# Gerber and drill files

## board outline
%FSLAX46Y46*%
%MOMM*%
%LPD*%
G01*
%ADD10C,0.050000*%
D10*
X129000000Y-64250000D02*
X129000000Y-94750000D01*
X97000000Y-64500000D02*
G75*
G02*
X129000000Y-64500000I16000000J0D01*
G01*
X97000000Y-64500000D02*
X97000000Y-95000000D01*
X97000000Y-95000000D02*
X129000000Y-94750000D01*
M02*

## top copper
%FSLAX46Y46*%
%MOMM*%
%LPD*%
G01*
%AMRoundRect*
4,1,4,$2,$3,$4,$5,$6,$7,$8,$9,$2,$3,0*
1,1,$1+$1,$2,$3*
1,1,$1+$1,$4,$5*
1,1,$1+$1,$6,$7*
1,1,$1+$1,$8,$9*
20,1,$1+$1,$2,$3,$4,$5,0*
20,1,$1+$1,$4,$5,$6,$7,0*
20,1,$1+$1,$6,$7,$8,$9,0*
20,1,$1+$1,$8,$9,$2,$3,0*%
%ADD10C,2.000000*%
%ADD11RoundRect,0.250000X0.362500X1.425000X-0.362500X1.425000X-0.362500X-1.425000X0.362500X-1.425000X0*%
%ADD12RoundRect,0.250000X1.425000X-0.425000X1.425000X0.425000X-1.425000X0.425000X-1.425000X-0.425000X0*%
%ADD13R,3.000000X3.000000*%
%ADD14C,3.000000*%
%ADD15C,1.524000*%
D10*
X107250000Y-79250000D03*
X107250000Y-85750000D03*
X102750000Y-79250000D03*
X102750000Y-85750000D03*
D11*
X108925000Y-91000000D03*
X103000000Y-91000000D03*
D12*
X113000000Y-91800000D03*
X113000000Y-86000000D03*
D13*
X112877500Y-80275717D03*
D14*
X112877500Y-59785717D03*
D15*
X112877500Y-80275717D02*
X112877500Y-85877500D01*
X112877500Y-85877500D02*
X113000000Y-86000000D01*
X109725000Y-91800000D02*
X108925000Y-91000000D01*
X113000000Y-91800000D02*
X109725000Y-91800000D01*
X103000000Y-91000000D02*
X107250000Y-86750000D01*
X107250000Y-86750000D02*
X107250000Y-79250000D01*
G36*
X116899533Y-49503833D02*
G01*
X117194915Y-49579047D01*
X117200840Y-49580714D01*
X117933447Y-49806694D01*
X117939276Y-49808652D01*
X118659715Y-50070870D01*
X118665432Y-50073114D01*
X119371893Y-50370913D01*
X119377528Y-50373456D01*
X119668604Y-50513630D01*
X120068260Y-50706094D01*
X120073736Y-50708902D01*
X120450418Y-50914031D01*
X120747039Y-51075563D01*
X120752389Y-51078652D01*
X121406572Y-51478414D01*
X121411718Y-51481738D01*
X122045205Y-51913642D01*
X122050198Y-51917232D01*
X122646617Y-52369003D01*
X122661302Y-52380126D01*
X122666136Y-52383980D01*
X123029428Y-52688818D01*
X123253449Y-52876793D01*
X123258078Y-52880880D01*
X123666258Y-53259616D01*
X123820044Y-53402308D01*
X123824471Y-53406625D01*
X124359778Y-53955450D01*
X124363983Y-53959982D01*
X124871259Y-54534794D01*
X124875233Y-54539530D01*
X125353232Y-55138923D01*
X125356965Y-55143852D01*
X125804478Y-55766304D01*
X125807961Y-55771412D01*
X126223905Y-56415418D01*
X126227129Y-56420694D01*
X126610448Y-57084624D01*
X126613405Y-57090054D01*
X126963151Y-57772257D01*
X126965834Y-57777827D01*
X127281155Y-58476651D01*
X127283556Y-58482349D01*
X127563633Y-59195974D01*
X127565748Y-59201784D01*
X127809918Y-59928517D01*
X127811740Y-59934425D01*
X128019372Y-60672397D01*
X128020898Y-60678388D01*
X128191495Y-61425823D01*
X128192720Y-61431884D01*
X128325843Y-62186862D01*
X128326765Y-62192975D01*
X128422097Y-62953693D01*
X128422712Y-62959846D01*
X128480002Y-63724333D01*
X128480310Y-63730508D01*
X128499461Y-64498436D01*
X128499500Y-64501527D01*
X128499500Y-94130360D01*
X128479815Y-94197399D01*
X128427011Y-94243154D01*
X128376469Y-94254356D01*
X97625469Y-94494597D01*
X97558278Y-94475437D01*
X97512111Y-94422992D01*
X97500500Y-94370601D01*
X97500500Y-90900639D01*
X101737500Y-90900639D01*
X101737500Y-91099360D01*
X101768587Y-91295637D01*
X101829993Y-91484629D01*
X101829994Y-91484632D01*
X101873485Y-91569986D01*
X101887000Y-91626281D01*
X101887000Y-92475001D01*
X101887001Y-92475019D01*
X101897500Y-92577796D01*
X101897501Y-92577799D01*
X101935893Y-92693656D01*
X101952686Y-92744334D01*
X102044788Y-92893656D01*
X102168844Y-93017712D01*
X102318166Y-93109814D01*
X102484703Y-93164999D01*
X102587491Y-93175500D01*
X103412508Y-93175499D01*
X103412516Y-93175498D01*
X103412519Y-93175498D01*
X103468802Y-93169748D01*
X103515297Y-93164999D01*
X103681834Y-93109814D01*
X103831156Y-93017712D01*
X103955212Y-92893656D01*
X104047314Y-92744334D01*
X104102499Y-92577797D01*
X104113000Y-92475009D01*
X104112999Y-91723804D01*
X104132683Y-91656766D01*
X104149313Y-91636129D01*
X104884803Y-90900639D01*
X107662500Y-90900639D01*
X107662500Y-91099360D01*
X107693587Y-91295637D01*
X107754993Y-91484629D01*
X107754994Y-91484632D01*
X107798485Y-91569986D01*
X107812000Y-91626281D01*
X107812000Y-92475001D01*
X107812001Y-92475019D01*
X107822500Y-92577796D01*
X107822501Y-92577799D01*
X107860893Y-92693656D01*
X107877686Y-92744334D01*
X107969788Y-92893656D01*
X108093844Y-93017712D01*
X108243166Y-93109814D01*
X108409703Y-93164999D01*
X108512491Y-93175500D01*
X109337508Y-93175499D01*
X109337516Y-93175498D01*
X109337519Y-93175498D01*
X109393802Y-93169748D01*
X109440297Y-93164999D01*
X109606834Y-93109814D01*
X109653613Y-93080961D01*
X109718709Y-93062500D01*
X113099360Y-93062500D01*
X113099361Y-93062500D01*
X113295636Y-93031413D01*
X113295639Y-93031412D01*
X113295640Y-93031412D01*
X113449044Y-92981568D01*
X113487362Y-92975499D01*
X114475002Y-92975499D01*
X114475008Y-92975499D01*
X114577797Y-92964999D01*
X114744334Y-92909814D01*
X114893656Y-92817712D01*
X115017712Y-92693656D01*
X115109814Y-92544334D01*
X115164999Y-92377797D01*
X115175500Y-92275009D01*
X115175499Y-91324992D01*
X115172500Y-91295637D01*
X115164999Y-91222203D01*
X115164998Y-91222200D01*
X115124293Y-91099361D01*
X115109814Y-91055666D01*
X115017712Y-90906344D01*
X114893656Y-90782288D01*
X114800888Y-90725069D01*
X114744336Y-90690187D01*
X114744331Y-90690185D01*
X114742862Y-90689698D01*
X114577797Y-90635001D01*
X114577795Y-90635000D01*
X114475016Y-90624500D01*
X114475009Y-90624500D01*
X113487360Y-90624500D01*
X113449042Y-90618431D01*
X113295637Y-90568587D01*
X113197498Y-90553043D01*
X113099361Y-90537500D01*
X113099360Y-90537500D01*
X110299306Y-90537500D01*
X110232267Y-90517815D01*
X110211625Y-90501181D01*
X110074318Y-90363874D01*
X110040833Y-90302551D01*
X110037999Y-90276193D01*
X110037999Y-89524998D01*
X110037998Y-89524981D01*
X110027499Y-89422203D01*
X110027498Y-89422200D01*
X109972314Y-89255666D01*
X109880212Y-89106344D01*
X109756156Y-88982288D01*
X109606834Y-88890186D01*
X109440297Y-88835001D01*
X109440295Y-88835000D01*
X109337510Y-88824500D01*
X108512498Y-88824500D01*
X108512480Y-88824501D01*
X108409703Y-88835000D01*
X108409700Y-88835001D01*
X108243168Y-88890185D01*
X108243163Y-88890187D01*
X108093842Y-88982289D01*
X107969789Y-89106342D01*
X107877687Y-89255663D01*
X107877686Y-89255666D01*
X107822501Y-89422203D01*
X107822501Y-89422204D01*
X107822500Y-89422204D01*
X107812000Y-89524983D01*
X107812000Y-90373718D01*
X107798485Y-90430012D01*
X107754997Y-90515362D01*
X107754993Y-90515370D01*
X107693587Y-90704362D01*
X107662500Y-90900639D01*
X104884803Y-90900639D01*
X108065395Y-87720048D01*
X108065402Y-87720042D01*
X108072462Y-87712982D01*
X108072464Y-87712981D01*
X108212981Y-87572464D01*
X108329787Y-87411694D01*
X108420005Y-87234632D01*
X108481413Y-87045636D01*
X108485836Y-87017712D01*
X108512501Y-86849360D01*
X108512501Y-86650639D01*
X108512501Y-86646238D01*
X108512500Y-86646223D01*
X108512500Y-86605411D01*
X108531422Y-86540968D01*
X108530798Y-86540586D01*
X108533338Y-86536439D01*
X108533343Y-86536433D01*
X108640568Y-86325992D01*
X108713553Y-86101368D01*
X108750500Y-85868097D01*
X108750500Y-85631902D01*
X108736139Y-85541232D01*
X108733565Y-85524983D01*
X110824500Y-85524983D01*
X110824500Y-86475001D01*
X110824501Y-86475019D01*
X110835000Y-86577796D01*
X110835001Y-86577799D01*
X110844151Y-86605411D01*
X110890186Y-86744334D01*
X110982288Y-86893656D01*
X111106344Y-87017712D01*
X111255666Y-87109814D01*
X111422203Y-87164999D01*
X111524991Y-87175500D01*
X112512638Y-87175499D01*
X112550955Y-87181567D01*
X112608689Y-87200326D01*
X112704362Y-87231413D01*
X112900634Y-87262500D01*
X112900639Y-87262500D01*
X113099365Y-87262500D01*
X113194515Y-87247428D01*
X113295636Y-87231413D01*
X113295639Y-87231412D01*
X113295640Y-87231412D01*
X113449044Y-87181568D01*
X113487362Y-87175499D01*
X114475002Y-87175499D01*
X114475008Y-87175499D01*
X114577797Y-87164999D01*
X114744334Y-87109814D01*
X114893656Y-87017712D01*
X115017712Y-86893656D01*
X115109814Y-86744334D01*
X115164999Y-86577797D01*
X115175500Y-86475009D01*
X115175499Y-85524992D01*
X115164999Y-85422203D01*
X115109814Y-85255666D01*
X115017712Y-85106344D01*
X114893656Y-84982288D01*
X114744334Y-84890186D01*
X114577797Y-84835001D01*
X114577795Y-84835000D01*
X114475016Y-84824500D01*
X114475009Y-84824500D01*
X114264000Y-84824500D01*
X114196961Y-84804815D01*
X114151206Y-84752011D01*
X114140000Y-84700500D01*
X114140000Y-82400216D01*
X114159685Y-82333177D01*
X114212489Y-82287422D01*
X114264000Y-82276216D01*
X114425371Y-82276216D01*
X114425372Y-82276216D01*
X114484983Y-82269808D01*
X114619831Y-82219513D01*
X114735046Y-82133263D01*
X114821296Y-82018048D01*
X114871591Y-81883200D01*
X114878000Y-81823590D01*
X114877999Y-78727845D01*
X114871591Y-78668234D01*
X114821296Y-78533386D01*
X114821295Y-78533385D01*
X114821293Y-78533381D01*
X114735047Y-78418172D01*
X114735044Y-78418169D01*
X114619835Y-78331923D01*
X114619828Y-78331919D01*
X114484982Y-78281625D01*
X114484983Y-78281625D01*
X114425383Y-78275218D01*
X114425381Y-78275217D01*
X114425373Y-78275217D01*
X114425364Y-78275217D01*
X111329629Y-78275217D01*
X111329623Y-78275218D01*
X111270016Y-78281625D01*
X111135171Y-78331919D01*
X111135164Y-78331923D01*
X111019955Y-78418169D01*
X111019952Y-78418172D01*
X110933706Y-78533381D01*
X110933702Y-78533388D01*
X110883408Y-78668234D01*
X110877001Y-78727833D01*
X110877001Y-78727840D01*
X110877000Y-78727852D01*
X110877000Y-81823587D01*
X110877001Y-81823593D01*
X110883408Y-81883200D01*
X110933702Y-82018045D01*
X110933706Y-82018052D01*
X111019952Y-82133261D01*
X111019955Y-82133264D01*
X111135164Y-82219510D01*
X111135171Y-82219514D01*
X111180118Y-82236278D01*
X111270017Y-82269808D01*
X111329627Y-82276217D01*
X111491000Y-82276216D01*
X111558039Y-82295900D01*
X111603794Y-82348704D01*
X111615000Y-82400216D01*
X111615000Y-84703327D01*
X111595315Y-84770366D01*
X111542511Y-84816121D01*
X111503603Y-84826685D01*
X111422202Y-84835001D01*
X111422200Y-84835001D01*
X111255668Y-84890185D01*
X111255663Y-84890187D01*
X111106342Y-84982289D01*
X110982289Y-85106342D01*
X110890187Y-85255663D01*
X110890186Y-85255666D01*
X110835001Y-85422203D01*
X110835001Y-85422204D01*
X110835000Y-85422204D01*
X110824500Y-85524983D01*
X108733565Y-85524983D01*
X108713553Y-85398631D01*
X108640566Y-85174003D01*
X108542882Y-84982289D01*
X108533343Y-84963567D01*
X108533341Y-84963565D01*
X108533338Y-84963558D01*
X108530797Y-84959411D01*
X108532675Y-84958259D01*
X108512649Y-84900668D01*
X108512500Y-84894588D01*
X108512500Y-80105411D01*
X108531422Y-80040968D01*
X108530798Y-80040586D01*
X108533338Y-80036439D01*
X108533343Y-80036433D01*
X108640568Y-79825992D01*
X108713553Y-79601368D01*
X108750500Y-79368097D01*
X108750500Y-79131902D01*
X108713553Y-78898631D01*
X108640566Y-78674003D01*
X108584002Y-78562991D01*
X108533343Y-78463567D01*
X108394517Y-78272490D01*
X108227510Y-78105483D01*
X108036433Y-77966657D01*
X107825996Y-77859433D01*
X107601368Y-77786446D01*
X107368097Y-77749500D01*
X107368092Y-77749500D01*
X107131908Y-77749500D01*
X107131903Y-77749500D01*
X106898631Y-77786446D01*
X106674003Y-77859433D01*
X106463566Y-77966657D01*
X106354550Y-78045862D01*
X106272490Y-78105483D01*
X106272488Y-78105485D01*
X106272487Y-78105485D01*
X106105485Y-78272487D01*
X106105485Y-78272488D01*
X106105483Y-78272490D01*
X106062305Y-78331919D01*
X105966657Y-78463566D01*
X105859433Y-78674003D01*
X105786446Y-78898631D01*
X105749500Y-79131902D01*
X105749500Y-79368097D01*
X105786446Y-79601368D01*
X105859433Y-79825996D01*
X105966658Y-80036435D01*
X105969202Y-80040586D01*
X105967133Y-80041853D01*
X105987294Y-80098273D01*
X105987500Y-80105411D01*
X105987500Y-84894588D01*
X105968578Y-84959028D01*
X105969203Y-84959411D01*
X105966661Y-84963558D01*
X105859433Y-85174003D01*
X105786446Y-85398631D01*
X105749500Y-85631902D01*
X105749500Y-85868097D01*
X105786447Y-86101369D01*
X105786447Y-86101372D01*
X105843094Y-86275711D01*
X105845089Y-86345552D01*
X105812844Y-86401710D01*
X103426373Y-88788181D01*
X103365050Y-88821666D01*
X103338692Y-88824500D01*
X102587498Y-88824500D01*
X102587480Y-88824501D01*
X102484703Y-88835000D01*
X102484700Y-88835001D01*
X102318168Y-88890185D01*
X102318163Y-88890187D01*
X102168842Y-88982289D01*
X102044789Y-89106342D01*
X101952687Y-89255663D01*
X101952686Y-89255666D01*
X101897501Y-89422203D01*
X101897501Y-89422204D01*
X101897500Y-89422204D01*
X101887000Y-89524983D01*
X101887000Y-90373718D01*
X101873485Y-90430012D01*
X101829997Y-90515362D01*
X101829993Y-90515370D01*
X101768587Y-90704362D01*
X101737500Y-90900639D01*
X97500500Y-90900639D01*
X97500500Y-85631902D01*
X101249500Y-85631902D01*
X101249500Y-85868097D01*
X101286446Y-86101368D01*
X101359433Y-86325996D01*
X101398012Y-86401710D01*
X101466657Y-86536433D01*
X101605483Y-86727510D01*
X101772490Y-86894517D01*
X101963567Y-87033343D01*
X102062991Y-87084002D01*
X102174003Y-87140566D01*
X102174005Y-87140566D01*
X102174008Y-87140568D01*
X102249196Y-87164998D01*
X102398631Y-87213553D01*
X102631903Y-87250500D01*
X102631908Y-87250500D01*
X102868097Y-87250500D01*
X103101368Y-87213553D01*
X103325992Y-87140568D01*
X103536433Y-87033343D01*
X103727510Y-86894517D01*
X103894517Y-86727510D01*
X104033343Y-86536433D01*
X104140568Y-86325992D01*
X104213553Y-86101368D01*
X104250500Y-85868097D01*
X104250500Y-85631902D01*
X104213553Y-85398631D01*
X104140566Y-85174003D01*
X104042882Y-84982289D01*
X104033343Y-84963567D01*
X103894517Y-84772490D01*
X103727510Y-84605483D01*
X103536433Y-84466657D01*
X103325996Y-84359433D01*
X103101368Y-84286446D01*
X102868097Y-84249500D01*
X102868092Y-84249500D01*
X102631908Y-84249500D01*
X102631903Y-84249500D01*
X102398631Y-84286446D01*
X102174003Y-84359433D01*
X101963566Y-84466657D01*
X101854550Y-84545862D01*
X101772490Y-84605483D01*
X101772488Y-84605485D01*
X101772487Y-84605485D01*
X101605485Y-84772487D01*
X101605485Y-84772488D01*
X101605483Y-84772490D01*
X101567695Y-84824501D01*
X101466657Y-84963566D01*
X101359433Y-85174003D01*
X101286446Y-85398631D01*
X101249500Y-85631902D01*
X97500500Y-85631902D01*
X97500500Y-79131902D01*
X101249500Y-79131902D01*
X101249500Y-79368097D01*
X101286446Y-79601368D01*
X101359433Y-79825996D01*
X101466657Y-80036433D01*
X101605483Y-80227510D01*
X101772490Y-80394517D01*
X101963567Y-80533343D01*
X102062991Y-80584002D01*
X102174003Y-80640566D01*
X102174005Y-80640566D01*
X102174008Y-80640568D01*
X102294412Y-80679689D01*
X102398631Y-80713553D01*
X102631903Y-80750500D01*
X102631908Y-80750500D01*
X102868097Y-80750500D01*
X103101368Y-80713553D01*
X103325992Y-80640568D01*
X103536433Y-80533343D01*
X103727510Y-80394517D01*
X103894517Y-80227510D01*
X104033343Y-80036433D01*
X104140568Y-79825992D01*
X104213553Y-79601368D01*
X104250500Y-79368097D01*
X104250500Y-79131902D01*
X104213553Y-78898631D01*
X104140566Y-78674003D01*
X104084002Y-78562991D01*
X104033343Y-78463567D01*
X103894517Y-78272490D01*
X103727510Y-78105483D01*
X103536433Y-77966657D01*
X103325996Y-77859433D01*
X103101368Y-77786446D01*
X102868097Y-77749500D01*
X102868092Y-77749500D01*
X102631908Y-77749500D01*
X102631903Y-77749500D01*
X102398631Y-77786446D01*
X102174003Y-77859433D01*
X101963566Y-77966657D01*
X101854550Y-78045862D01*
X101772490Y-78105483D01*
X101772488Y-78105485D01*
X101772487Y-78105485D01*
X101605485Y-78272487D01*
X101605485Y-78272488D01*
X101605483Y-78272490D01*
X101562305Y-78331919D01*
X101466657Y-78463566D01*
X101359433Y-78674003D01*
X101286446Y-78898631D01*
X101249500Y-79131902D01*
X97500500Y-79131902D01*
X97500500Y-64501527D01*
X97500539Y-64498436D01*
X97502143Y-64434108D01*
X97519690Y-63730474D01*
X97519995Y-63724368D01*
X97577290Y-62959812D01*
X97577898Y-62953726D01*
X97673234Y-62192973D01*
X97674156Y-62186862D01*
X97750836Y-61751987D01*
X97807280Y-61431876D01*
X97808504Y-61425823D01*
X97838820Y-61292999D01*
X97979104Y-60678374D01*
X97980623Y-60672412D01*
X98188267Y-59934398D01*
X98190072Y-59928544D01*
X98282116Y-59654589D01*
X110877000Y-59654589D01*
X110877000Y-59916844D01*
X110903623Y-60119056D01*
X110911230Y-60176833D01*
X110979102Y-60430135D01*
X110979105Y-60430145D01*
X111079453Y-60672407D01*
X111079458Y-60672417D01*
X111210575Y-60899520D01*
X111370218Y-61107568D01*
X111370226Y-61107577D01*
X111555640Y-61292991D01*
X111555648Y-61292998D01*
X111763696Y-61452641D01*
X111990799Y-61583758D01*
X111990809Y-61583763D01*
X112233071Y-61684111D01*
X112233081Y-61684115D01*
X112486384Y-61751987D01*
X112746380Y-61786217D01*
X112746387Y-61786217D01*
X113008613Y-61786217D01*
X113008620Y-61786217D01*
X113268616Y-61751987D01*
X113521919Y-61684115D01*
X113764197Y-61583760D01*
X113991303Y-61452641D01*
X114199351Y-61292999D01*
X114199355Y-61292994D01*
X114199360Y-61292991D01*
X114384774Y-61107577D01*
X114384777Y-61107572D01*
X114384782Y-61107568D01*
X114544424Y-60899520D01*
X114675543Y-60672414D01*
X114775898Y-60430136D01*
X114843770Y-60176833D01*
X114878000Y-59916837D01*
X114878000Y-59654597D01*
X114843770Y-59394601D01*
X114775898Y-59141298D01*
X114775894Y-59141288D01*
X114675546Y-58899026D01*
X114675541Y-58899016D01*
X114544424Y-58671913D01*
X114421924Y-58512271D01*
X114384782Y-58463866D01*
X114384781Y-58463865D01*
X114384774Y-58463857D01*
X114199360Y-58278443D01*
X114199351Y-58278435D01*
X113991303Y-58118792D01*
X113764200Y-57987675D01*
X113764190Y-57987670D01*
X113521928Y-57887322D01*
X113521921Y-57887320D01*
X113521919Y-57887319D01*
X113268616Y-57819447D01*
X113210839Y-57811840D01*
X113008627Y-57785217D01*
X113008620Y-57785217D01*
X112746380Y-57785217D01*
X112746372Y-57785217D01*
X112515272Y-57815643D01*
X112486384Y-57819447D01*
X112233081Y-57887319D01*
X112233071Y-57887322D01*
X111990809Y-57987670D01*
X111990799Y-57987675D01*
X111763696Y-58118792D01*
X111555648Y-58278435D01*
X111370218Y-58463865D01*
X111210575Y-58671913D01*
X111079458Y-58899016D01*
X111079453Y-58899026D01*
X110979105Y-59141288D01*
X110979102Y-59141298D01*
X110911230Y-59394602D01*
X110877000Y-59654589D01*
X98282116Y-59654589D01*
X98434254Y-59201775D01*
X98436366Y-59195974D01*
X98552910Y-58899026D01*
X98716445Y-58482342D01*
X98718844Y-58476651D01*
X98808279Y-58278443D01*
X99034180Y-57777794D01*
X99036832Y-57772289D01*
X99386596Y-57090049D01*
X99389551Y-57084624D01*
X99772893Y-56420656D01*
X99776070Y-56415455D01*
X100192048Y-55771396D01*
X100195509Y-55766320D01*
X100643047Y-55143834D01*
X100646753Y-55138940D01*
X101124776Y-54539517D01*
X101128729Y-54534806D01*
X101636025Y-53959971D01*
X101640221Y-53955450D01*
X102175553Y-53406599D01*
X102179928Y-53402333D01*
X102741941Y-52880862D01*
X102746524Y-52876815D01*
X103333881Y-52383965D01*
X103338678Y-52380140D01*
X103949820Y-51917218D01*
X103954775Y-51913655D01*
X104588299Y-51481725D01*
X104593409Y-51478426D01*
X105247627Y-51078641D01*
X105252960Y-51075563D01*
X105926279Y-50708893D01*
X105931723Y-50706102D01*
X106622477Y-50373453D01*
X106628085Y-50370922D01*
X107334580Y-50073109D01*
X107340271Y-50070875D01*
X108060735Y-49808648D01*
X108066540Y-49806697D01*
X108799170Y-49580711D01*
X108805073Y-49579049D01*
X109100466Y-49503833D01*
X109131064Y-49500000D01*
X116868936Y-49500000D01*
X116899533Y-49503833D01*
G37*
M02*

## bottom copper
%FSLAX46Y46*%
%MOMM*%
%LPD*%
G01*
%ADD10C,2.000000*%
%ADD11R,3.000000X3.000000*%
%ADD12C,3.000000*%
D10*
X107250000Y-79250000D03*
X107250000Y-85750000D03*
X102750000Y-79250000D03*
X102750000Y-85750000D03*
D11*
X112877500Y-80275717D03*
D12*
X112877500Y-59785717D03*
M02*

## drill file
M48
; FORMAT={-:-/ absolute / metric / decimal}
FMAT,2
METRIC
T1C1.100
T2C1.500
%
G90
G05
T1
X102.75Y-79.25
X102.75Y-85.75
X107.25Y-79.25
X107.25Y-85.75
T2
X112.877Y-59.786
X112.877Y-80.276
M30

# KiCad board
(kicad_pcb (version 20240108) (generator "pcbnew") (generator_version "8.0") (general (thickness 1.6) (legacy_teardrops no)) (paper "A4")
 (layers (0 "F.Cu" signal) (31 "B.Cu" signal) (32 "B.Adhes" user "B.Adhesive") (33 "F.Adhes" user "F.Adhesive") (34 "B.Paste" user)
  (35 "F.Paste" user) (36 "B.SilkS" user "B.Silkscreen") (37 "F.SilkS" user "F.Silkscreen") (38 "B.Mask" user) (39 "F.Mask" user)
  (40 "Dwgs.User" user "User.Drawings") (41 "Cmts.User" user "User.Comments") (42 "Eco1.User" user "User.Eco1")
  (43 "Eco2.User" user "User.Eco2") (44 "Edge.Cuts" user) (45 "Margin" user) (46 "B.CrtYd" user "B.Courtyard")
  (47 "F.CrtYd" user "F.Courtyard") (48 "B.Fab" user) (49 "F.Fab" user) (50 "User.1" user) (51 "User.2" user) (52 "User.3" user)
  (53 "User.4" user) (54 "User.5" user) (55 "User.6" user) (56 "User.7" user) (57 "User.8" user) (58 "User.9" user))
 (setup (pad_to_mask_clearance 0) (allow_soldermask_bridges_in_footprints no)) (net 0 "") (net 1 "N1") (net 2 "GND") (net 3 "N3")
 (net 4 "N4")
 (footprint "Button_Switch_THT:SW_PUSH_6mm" (layer "F.Cu") (at 107.25 79.25 -90)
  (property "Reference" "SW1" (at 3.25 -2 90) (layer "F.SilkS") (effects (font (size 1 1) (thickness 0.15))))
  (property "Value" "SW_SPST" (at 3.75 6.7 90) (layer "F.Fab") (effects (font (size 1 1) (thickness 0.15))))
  (pad "1" thru_hole circle (at 0 0) (size 2 2) (drill 1.1) (layers "*.Cu" "*.Mask") (remove_unused_layers no) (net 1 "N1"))
  (pad "1" thru_hole circle (at 6.5 0) (size 2 2) (drill 1.1) (layers "*.Cu" "*.Mask") (remove_unused_layers no) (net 1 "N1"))
  (pad "2" thru_hole circle (at 0 4.5) (size 2 2) (drill 1.1) (layers "*.Cu" "*.Mask") (remove_unused_layers no) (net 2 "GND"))
  (pad "2" thru_hole circle (at 6.5 4.5) (size 2 2) (drill 1.1) (layers "*.Cu" "*.Mask") (remove_unused_layers no) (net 2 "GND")))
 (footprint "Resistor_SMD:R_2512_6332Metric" (layer "F.Cu") (at 105.9625 91 180)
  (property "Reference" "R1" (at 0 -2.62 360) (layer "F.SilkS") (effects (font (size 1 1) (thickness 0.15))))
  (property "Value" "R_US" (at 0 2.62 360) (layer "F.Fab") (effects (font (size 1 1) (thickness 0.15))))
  (pad "1" smd roundrect (at -2.9625 0 180) (size 1.225 3.35) (layers "F.Cu" "F.Paste" "F.Mask") (roundrect_rratio 0.204082) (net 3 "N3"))
  (pad "2" smd roundrect (at 2.9625 0 180) (size 1.225 3.35) (layers "F.Cu" "F.Paste" "F.Mask") (roundrect_rratio 0.204082) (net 1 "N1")))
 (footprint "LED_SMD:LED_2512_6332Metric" (layer "F.Cu") (at 113 88.9 90)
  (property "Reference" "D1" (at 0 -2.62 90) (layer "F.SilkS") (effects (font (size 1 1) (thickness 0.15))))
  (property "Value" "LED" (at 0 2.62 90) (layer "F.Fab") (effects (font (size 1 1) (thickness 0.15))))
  (pad "1" smd roundrect (at -2.9 0 90) (size 1.35 3.35) (layers "F.Cu" "F.Paste" "F.Mask") (roundrect_rratio 0.185185) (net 3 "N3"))
  (pad "2" smd roundrect (at 2.9 0 90) (size 1.35 3.35) (layers "F.Cu" "F.Paste" "F.Mask") (roundrect_rratio 0.185185) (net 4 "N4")))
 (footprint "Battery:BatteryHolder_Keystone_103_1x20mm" (layer "F.Cu") (at 112.8775 80.275717 90)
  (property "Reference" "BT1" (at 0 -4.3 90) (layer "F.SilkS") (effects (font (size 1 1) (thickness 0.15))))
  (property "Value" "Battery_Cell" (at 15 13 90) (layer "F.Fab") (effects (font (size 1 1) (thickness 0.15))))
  (pad "1" thru_hole rect (at 0 0 90) (size 3 3) (drill 1.5) (layers "*.Cu" "*.Mask") (remove_unused_layers no) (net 4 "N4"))
  (pad "2" thru_hole circle (at 20.49 0 90) (size 3 3) (drill 1.5) (layers "*.Cu" "*.Mask") (remove_unused_layers no) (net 2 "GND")))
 (gr_line (start 129 64.25) (end 129 94.75) (stroke (width 0.05) (type default)) (layer "Edge.Cuts"))
 (gr_arc (start 97 64.5) (mid 113 48.5) (end 129 64.5) (stroke (width 0.05) (type default)) (layer "Edge.Cuts"))
 (gr_line (start 97 64.5) (end 97 95) (stroke (width 0.05) (type default)) (layer "Edge.Cuts"))
 (gr_line (start 97 95) (end 129 94.75) (stroke (width 0.05) (type default)) (layer "Edge.Cuts"))
 (segment (start 112.8775 80.275717) (end 112.8775 85.8775) (width 1.524) (layer "F.Cu") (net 4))
 (segment (start 112.8775 85.8775) (end 113 86) (width 1.524) (layer "F.Cu") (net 4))
 (segment (start 109.725 91.8) (end 108.925 91) (width 1.524) (layer "F.Cu") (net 3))
 (segment (start 113 91.8) (end 109.725 91.8) (width 1.524) (layer "F.Cu") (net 3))
 (segment (start 103 91) (end 107.25 86.75) (width 1.524) (layer "F.Cu") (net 1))
 (segment (start 107.25 86.75) (end 107.25 79.25) (width 1.524) (layer "F.Cu") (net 1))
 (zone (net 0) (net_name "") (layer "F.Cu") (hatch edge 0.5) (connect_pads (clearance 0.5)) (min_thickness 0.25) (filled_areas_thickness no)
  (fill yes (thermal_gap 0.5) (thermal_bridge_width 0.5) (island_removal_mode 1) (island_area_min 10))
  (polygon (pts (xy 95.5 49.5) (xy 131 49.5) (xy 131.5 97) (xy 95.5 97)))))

